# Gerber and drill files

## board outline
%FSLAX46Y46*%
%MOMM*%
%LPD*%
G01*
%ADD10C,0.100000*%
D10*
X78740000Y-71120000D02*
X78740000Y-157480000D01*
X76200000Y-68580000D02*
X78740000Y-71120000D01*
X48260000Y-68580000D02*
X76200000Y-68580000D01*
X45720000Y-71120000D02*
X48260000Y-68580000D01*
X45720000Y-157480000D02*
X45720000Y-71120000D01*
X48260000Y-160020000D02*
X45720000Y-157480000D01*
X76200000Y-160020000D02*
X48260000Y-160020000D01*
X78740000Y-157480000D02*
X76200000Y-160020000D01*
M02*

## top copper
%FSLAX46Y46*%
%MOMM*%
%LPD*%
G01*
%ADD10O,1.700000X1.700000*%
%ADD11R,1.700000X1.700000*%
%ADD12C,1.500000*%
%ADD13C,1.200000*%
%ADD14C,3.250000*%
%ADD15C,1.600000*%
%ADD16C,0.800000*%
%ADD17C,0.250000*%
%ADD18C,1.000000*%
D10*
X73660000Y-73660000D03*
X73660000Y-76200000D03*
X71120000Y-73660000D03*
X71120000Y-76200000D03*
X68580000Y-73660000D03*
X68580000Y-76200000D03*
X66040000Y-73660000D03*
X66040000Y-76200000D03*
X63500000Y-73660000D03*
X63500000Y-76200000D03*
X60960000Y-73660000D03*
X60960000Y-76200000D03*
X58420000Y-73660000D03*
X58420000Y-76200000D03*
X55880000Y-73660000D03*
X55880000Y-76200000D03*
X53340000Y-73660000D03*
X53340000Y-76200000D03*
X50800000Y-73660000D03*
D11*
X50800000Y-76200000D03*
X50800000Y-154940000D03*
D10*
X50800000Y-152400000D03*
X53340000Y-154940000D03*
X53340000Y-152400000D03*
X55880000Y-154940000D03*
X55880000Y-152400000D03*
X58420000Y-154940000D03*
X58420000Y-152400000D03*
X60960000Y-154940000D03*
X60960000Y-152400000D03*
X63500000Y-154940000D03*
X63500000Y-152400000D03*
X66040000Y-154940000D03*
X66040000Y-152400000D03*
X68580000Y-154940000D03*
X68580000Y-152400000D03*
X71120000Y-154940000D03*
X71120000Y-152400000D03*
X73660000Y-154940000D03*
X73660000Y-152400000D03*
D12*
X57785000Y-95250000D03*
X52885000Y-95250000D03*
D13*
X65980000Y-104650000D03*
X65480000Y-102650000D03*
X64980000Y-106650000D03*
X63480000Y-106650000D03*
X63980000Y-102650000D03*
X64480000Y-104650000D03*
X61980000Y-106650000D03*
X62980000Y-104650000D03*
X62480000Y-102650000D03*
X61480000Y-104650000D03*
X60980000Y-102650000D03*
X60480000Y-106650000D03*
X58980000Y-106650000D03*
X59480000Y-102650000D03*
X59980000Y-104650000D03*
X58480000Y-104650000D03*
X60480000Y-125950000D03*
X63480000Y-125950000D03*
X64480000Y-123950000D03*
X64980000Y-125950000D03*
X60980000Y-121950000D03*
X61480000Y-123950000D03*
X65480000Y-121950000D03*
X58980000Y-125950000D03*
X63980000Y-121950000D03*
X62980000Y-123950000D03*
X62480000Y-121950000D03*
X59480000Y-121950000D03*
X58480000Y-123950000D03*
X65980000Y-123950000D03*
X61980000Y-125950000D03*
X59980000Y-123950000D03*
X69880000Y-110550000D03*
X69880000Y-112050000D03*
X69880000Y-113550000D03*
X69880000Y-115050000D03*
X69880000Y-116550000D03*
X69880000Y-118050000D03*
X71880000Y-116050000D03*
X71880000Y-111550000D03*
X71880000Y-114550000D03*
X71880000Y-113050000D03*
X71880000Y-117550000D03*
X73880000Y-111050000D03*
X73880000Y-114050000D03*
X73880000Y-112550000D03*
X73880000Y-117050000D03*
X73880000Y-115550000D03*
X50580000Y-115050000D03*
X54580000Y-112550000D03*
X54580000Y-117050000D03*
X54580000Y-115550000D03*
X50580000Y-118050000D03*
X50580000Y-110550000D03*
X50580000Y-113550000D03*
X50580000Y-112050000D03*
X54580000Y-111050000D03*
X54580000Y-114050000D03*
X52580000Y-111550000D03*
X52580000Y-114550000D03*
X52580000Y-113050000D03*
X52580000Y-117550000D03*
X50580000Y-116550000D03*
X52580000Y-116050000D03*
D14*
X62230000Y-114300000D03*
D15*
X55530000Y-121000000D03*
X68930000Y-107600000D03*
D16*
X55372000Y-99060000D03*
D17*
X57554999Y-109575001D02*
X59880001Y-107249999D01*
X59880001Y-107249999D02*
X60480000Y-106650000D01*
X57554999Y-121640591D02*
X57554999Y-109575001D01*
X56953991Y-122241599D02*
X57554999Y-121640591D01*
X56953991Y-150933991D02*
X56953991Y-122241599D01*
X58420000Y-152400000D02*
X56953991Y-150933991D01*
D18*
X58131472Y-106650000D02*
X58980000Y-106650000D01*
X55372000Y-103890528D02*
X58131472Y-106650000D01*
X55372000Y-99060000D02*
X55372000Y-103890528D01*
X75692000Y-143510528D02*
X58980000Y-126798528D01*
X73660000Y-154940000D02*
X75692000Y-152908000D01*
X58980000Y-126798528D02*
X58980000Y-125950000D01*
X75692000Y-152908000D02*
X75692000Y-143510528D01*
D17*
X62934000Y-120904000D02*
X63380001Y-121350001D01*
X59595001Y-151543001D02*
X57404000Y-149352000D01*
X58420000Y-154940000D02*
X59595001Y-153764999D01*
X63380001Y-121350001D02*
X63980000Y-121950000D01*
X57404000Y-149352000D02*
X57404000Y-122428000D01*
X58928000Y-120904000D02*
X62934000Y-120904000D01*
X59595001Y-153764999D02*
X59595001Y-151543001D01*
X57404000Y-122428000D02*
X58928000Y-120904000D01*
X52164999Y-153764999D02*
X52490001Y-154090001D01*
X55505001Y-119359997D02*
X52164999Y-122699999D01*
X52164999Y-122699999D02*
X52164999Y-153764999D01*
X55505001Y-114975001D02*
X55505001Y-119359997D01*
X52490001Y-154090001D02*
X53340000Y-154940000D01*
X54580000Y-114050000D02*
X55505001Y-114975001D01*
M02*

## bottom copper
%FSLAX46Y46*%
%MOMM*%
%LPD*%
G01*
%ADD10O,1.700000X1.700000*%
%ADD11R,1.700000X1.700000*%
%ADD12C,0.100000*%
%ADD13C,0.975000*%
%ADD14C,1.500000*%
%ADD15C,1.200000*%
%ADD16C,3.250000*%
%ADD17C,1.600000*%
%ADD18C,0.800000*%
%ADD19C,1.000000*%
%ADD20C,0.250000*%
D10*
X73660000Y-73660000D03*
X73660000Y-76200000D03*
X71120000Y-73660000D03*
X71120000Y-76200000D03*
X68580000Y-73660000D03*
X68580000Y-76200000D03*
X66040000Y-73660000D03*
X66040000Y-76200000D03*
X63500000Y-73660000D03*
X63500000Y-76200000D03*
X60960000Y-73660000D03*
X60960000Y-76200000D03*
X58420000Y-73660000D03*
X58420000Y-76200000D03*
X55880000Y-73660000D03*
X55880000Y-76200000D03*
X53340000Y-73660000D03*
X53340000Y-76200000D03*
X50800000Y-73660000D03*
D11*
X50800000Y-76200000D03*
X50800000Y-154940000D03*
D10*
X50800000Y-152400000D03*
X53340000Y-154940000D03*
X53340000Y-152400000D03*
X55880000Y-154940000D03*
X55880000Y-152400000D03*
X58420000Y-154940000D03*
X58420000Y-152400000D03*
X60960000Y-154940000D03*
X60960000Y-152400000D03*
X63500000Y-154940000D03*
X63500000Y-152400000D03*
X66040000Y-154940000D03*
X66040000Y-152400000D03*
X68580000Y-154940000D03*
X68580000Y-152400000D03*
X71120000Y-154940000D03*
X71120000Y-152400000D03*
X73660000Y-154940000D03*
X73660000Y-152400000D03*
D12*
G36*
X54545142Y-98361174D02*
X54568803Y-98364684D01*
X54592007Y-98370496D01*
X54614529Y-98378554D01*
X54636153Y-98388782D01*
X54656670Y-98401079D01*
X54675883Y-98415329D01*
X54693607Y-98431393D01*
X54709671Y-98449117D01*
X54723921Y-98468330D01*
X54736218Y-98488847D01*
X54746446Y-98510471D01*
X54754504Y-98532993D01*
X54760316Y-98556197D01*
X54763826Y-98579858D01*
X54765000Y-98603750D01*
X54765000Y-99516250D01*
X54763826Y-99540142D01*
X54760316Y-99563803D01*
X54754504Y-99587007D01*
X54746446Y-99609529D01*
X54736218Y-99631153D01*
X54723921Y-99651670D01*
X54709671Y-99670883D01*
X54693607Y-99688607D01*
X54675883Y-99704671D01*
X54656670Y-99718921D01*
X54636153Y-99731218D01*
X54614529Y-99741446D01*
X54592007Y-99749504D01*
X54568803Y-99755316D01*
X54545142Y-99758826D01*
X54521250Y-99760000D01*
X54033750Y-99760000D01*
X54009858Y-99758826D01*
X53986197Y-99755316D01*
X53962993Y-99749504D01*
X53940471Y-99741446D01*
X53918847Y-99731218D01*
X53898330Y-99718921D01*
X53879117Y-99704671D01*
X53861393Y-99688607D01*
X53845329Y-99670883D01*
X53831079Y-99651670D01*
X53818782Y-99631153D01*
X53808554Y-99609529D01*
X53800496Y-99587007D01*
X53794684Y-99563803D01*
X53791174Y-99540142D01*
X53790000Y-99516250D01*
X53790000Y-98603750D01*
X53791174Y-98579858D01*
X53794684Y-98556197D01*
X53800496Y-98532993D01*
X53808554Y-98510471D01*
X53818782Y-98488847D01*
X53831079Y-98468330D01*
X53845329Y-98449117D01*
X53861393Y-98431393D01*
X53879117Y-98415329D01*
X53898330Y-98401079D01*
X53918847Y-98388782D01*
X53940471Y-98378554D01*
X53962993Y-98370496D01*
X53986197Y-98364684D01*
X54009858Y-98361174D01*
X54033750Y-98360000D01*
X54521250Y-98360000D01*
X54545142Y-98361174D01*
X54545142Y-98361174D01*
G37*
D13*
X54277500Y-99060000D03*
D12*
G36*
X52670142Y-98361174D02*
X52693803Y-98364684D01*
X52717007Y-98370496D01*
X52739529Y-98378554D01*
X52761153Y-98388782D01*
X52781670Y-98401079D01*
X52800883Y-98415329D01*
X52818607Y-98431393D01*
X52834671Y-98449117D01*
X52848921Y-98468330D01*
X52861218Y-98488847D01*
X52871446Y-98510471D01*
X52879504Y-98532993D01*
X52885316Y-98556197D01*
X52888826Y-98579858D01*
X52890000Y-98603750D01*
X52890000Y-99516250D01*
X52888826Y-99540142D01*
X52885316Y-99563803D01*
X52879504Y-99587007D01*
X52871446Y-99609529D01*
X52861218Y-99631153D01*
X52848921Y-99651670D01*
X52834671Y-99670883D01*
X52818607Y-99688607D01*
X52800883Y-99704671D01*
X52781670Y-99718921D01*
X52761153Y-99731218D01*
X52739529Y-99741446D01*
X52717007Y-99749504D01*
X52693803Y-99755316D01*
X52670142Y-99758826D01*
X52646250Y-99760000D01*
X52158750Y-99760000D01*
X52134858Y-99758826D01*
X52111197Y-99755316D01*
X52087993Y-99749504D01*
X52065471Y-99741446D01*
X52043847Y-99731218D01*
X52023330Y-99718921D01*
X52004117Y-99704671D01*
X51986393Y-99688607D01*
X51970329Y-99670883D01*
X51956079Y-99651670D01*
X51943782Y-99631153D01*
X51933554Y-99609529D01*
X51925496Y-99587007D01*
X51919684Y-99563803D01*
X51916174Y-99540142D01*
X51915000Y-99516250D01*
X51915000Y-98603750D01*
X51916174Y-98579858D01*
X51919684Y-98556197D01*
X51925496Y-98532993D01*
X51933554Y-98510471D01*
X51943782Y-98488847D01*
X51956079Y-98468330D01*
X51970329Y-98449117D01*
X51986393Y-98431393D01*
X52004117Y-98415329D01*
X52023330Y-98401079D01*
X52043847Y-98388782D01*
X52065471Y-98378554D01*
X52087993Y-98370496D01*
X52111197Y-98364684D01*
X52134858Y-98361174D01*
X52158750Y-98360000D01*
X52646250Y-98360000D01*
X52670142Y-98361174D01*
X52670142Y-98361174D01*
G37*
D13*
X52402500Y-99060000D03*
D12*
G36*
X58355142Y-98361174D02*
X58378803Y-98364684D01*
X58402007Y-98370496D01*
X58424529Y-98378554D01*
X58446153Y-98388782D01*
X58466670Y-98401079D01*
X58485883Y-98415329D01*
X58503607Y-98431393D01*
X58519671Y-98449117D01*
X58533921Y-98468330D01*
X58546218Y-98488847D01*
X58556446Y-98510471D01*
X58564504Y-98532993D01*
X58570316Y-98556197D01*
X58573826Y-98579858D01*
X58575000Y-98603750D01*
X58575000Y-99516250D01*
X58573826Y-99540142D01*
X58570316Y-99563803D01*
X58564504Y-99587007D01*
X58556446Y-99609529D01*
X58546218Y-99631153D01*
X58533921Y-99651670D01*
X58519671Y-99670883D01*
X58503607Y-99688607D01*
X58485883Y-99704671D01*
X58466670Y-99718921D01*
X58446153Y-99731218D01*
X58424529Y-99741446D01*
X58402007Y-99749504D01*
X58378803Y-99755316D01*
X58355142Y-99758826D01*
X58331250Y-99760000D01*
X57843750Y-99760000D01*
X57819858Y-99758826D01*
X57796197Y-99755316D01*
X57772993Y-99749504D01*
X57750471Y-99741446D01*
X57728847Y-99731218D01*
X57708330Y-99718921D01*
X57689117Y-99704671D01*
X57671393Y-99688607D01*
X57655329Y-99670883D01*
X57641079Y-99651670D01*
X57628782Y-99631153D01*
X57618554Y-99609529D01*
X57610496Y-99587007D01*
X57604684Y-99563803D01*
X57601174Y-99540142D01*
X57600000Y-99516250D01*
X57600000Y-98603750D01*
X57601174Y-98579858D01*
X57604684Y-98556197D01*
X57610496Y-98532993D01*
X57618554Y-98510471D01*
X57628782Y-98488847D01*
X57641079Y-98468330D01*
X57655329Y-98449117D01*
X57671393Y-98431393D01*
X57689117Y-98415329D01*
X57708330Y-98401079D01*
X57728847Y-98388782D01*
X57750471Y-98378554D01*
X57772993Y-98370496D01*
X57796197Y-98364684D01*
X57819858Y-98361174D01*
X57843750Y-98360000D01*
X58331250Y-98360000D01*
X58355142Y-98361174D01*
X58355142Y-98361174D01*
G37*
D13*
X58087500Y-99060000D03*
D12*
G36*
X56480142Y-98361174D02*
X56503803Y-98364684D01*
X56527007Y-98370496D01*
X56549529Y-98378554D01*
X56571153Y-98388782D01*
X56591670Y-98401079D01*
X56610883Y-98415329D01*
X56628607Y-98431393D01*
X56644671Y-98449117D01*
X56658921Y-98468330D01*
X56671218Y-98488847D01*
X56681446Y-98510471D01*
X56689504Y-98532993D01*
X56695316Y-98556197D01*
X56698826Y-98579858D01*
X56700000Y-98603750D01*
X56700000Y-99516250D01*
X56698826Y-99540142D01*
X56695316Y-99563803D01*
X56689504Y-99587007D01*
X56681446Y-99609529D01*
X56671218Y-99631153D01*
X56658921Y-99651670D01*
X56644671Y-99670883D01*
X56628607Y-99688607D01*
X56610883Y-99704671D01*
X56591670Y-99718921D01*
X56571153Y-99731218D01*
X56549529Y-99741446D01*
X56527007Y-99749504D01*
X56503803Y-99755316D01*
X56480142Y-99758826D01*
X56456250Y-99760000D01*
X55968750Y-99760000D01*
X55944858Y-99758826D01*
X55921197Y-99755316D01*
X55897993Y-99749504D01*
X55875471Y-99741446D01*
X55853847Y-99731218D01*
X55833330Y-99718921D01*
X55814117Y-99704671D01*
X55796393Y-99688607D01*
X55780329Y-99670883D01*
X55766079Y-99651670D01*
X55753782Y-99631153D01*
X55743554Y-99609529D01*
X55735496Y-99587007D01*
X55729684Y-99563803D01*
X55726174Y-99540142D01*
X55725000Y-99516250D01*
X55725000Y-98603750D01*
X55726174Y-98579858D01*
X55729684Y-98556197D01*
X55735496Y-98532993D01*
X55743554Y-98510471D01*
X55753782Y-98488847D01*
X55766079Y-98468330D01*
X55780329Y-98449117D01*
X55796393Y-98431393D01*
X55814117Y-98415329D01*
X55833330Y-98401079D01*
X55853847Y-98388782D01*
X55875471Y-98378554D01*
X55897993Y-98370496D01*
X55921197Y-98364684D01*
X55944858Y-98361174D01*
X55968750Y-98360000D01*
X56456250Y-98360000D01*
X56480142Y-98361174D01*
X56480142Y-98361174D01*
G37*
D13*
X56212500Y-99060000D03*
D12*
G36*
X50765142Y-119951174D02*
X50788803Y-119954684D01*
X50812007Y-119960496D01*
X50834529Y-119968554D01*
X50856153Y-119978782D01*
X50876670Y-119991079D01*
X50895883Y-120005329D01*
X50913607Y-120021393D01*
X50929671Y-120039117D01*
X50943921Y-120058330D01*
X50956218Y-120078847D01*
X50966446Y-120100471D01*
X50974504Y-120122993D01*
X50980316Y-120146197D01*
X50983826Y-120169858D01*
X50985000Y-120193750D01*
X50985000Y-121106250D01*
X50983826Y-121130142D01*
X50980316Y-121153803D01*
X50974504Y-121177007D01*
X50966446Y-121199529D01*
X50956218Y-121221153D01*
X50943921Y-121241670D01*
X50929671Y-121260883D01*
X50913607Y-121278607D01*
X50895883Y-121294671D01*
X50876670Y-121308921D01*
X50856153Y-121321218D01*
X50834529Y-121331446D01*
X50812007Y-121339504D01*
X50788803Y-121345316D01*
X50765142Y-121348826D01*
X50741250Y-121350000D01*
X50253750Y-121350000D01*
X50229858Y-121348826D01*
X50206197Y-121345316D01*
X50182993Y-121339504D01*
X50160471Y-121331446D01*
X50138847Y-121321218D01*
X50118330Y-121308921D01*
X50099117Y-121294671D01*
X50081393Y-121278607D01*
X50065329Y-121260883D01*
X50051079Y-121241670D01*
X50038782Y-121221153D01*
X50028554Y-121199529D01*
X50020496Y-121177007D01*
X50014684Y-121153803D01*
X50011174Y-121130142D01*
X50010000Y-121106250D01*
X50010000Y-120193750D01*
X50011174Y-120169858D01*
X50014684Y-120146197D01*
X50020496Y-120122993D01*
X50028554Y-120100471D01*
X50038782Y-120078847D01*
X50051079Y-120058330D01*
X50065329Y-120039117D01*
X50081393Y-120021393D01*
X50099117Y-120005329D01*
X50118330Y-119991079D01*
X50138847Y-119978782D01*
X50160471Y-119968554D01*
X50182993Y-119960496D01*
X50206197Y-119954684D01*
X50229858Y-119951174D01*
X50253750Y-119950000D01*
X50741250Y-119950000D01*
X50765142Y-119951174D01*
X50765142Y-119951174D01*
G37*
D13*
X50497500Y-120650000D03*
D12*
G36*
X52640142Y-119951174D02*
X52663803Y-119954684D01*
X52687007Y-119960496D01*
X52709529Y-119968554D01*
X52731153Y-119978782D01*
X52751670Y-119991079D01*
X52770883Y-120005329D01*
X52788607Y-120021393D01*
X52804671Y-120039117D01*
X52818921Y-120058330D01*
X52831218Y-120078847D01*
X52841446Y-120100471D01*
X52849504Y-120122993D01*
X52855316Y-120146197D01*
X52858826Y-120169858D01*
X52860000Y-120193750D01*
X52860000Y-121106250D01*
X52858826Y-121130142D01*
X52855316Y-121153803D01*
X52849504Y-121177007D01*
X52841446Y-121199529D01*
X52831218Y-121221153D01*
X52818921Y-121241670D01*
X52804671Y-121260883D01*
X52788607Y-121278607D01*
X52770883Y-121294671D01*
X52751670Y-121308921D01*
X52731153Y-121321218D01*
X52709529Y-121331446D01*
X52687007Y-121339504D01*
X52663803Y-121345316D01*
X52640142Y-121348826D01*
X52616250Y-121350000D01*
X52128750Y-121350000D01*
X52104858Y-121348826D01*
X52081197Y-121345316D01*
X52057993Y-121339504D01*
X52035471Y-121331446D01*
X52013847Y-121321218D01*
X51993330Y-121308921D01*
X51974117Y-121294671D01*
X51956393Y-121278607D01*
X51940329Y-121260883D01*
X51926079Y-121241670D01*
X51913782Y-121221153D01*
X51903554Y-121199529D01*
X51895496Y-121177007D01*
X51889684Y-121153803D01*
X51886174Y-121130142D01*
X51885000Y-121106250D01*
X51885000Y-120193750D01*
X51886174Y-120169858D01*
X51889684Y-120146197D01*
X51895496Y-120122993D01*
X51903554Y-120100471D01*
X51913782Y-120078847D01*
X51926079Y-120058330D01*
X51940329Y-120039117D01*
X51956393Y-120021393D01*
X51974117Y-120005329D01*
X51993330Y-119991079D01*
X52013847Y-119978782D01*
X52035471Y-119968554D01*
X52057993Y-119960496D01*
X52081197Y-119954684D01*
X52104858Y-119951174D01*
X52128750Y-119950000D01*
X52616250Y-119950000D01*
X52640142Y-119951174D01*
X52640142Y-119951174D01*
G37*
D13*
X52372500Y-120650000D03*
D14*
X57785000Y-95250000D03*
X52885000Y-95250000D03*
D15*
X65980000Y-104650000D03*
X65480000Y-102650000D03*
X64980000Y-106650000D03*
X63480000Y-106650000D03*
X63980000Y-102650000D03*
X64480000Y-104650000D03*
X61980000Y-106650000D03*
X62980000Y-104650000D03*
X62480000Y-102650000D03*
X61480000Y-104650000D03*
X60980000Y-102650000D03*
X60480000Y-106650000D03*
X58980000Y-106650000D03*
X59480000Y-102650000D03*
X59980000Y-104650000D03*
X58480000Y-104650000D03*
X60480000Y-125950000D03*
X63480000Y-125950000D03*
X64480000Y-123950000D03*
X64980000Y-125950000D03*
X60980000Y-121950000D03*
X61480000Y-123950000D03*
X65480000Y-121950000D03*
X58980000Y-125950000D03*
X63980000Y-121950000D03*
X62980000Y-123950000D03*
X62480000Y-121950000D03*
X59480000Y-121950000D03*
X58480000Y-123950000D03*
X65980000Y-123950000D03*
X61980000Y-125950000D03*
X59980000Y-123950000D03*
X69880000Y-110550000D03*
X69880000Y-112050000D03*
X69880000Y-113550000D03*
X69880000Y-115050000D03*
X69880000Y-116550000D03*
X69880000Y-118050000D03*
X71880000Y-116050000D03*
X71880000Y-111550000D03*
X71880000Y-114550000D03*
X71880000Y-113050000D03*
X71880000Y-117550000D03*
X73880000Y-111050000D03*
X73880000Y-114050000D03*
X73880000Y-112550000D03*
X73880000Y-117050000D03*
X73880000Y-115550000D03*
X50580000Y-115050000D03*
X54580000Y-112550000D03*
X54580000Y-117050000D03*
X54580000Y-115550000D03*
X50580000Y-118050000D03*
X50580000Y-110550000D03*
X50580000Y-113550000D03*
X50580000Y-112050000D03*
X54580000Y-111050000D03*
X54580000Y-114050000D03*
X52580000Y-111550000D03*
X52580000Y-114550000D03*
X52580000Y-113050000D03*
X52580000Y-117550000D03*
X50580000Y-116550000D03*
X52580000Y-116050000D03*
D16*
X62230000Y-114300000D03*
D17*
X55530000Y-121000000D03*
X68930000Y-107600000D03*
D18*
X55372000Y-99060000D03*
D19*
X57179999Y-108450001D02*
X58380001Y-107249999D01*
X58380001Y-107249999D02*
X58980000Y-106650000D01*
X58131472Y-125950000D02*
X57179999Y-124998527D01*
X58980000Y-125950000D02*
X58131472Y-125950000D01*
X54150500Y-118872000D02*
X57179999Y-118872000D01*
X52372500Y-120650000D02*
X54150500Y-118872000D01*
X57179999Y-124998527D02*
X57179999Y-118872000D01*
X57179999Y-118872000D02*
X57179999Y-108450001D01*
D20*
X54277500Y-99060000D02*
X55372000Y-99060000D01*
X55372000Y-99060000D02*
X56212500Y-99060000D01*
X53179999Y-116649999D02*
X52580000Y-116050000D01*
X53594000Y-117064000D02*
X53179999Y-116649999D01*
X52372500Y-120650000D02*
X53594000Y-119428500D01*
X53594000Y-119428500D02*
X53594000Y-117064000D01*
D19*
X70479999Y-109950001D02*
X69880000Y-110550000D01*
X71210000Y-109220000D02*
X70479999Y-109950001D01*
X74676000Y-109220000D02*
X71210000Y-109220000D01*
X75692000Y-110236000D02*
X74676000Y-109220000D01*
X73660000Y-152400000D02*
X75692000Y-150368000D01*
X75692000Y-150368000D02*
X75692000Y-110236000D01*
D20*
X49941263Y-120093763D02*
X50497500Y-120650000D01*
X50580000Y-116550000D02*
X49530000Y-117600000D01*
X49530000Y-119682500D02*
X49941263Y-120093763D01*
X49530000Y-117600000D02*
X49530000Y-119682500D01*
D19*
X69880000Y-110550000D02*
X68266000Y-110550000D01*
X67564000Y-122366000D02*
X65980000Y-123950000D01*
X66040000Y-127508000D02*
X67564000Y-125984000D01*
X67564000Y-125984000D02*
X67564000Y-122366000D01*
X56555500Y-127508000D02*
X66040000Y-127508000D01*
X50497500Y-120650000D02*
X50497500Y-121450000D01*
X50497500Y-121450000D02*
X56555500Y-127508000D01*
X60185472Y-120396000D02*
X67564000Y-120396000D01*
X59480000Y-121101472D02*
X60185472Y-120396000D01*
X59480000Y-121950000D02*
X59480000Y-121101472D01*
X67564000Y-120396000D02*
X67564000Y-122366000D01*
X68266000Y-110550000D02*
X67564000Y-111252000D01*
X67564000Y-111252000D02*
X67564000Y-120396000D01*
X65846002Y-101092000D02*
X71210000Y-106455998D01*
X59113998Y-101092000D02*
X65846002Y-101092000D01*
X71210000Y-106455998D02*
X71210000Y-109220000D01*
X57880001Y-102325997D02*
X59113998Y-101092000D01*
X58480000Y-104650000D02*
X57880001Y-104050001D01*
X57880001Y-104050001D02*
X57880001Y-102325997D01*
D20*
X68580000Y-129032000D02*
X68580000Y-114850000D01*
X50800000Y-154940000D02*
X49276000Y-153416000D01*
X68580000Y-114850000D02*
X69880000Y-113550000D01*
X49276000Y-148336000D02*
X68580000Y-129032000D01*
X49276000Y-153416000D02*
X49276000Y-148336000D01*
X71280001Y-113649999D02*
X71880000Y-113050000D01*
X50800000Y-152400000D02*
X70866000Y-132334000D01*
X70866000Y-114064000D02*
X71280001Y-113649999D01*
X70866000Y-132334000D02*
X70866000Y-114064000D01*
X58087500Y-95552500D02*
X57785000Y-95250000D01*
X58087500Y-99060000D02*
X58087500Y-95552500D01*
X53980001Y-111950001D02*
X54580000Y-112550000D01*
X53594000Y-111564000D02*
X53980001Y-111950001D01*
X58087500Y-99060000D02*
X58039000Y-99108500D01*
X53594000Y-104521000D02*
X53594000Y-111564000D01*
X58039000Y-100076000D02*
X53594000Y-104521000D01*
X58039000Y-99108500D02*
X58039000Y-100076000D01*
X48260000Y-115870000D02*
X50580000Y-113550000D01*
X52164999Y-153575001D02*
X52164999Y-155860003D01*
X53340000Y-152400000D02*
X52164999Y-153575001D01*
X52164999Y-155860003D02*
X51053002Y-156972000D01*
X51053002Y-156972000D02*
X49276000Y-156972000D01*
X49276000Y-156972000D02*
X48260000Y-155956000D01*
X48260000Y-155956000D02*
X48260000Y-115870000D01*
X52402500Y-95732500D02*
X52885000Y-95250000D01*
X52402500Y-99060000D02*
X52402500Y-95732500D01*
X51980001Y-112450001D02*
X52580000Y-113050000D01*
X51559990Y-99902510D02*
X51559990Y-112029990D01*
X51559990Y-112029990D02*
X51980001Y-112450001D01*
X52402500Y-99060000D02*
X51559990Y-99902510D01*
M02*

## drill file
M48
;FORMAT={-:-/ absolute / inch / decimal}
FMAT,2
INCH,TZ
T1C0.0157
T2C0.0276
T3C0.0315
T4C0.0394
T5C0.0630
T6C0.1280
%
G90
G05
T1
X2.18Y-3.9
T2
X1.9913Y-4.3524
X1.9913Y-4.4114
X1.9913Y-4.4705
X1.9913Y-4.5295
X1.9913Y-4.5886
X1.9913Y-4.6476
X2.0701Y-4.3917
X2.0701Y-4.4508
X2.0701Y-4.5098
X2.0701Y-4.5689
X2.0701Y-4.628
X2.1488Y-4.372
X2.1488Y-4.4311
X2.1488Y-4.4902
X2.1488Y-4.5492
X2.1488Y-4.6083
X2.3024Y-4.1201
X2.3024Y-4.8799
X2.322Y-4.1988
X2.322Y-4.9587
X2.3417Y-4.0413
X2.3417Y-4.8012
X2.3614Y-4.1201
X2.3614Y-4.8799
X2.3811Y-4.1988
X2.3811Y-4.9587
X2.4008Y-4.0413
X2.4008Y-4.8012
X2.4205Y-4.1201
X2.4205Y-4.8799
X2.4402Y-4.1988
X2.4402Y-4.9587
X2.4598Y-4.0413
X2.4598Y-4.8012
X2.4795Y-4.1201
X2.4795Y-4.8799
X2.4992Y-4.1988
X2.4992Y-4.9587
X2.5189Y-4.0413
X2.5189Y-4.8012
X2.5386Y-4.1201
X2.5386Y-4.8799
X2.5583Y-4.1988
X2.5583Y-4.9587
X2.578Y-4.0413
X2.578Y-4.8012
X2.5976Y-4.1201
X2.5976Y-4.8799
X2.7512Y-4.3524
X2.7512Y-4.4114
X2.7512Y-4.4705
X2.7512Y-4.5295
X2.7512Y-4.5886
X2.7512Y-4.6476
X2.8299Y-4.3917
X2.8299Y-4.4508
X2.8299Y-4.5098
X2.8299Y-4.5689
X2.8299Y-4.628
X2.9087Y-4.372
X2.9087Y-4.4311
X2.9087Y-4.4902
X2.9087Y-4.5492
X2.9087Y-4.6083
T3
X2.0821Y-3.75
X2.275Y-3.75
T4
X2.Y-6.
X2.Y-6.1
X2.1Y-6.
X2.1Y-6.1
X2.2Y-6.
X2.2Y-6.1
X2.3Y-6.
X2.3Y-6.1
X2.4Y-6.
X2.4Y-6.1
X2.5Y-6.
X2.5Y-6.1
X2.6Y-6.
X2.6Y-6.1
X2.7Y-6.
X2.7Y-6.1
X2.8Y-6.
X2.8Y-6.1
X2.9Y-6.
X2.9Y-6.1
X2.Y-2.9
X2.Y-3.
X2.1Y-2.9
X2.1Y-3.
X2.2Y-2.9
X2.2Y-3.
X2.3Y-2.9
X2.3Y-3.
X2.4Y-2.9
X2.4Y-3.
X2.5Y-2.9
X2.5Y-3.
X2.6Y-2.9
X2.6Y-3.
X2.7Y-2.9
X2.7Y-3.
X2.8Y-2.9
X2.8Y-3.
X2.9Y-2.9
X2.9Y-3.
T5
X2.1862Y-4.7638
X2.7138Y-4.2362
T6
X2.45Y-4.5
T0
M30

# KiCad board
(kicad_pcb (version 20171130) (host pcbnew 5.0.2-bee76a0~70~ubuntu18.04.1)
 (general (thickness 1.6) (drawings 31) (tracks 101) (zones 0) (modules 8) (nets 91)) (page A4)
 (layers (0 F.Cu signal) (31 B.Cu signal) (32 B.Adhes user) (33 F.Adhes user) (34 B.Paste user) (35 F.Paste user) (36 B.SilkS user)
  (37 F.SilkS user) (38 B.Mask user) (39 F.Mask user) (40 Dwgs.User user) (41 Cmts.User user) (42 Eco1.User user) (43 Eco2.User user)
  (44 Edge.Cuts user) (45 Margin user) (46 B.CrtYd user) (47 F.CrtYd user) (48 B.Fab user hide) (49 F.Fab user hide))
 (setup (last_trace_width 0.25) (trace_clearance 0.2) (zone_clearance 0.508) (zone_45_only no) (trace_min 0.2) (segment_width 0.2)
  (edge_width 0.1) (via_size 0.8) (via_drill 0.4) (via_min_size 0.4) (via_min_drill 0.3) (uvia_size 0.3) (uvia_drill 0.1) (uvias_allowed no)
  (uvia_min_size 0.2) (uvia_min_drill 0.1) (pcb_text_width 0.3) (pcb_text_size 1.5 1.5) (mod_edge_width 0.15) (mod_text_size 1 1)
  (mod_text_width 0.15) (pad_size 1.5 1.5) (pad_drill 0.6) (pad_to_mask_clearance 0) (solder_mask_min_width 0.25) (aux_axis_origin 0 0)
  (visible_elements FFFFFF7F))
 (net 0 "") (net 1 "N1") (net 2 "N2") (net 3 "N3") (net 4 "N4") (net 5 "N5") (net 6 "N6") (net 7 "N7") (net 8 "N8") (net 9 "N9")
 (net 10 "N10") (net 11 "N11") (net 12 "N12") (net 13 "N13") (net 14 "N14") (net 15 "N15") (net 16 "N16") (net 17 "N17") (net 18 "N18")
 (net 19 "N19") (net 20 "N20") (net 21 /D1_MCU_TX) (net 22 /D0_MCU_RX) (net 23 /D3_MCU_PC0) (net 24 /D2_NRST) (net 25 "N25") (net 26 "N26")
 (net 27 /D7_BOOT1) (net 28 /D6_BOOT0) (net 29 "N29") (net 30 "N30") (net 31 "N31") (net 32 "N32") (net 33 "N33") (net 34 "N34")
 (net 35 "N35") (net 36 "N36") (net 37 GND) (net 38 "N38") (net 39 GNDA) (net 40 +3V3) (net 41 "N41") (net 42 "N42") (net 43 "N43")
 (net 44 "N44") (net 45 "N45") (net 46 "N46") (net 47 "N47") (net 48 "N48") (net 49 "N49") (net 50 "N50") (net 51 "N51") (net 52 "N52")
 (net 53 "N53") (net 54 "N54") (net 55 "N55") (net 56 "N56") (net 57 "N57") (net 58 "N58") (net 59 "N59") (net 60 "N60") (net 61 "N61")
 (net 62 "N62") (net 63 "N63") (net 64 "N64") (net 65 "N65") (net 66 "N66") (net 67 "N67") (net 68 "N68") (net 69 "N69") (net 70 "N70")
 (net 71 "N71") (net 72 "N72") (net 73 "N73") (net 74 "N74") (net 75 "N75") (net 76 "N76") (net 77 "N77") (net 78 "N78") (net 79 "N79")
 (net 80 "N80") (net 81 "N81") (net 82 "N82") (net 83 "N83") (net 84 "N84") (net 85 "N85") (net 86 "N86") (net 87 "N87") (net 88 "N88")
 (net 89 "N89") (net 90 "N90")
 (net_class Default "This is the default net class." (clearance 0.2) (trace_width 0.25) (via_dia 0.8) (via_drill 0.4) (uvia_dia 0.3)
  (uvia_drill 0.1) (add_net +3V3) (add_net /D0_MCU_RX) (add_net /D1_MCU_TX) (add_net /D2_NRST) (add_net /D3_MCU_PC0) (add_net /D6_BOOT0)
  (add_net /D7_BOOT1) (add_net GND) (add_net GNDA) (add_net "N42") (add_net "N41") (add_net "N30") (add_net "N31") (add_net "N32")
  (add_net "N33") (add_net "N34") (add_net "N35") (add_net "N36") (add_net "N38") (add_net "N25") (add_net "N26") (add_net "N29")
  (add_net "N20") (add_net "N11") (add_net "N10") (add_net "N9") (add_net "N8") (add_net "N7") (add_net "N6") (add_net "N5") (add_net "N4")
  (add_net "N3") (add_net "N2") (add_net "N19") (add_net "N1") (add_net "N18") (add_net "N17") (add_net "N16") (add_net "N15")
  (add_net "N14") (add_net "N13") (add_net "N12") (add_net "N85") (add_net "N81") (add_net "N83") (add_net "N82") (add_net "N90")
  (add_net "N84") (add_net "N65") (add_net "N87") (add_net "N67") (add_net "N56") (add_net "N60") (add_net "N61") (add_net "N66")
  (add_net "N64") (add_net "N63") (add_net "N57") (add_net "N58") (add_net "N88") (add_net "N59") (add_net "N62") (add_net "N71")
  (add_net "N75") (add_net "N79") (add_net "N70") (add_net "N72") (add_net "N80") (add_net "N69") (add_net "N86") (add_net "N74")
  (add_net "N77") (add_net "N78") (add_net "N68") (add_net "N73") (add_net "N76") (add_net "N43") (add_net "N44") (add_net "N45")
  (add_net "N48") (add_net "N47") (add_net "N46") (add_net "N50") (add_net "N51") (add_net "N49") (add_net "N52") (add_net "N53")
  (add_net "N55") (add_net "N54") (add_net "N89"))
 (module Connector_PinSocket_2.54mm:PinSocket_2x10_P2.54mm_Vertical (layer B.Cu) (at 50.8 76.2 270)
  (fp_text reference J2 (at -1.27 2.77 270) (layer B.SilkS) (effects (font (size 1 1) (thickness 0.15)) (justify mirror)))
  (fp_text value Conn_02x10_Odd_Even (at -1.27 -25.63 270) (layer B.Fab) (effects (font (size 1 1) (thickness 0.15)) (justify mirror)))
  (pad 20 thru_hole oval (at -2.54 -22.86 270) (size 1.7 1.7) (drill 1) (layers *.Cu *.Mask) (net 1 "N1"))
  (pad 19 thru_hole oval (at 0 -22.86 270) (size 1.7 1.7) (drill 1) (layers *.Cu *.Mask) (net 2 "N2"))
  (pad 18 thru_hole oval (at -2.54 -20.32 270) (size 1.7 1.7) (drill 1) (layers *.Cu *.Mask) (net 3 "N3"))
  (pad 17 thru_hole oval (at 0 -20.32 270) (size 1.7 1.7) (drill 1) (layers *.Cu *.Mask) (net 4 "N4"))
  (pad 16 thru_hole oval (at -2.54 -17.78 270) (size 1.7 1.7) (drill 1) (layers *.Cu *.Mask) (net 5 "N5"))
  (pad 15 thru_hole oval (at 0 -17.78 270) (size 1.7 1.7) (drill 1) (layers *.Cu *.Mask) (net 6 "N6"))
  (pad 14 thru_hole oval (at -2.54 -15.24 270) (size 1.7 1.7) (drill 1) (layers *.Cu *.Mask) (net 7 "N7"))
  (pad 13 thru_hole oval (at 0 -15.24 270) (size 1.7 1.7) (drill 1) (layers *.Cu *.Mask) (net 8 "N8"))
  (pad 12 thru_hole oval (at -2.54 -12.7 270) (size 1.7 1.7) (drill 1) (layers *.Cu *.Mask) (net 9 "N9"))
  (pad 11 thru_hole oval (at 0 -12.7 270) (size 1.7 1.7) (drill 1) (layers *.Cu *.Mask) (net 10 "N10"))
  (pad 10 thru_hole oval (at -2.54 -10.16 270) (size 1.7 1.7) (drill 1) (layers *.Cu *.Mask) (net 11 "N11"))
  (pad 9 thru_hole oval (at 0 -10.16 270) (size 1.7 1.7) (drill 1) (layers *.Cu *.Mask) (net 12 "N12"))
  (pad 8 thru_hole oval (at -2.54 -7.62 270) (size 1.7 1.7) (drill 1) (layers *.Cu *.Mask) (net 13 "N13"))
  (pad 7 thru_hole oval (at 0 -7.62 270) (size 1.7 1.7) (drill 1) (layers *.Cu *.Mask) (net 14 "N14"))
  (pad 6 thru_hole oval (at -2.54 -5.08 270) (size 1.7 1.7) (drill 1) (layers *.Cu *.Mask) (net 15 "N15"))
  (pad 5 thru_hole oval (at 0 -5.08 270) (size 1.7 1.7) (drill 1) (layers *.Cu *.Mask) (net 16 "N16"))
  (pad 4 thru_hole oval (at -2.54 -2.54 270) (size 1.7 1.7) (drill 1) (layers *.Cu *.Mask) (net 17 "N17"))
  (pad 3 thru_hole oval (at 0 -2.54 270) (size 1.7 1.7) (drill 1) (layers *.Cu *.Mask) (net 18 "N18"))
  (pad 2 thru_hole oval (at -2.54 0 270) (size 1.7 1.7) (drill 1) (layers *.Cu *.Mask) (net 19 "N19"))
  (pad 1 thru_hole rect (at 0 0 270) (size 1.7 1.7) (drill 1) (layers *.Cu *.Mask) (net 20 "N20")))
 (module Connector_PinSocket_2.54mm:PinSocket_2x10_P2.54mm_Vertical (layer B.Cu) (at 50.8 154.94 270)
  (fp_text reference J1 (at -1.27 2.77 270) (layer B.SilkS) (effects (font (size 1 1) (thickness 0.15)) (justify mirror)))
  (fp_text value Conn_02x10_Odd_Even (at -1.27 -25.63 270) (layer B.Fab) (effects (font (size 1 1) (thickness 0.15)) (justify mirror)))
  (pad 1 thru_hole rect (at 0 0 270) (size 1.7 1.7) (drill 1) (layers *.Cu *.Mask) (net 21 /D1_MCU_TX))
  (pad 2 thru_hole oval (at -2.54 0 270) (size 1.7 1.7) (drill 1) (layers *.Cu *.Mask) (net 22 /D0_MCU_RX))
  (pad 3 thru_hole oval (at 0 -2.54 270) (size 1.7 1.7) (drill 1) (layers *.Cu *.Mask) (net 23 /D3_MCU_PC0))
  (pad 4 thru_hole oval (at -2.54 -2.54 270) (size 1.7 1.7) (drill 1) (layers *.Cu *.Mask) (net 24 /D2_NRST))
  (pad 5 thru_hole oval (at 0 -5.08 270) (size 1.7 1.7) (drill 1) (layers *.Cu *.Mask) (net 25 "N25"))
  (pad 6 thru_hole oval (at -2.54 -5.08 270) (size 1.7 1.7) (drill 1) (layers *.Cu *.Mask) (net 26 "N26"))
  (pad 7 thru_hole oval (at 0 -7.62 270) (size 1.7 1.7) (drill 1) (layers *.Cu *.Mask) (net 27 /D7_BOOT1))
  (pad 8 thru_hole oval (at -2.54 -7.62 270) (size 1.7 1.7) (drill 1) (layers *.Cu *.Mask) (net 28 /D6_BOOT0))
  (pad 9 thru_hole oval (at 0 -10.16 270) (size 1.7 1.7) (drill 1) (layers *.Cu *.Mask) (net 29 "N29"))
  (pad 10 thru_hole oval (at -2.54 -10.16 270) (size 1.7 1.7) (drill 1) (layers *.Cu *.Mask) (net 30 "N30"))
  (pad 11 thru_hole oval (at 0 -12.7 270) (size 1.7 1.7) (drill 1) (layers *.Cu *.Mask) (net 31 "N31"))
  (pad 12 thru_hole oval (at -2.54 -12.7 270) (size 1.7 1.7) (drill 1) (layers *.Cu *.Mask) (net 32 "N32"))
  (pad 13 thru_hole oval (at 0 -15.24 270) (size 1.7 1.7) (drill 1) (layers *.Cu *.Mask) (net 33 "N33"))
  (pad 14 thru_hole oval (at -2.54 -15.24 270) (size 1.7 1.7) (drill 1) (layers *.Cu *.Mask) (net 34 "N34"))
  (pad 15 thru_hole oval (at 0 -17.78 270) (size 1.7 1.7) (drill 1) (layers *.Cu *.Mask) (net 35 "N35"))
  (pad 16 thru_hole oval (at -2.54 -17.78 270) (size 1.7 1.7) (drill 1) (layers *.Cu *.Mask) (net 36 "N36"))
  (pad 17 thru_hole oval (at 0 -20.32 270) (size 1.7 1.7) (drill 1) (layers *.Cu *.Mask) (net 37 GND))
  (pad 18 thru_hole oval (at -2.54 -20.32 270) (size 1.7 1.7) (drill 1) (layers *.Cu *.Mask) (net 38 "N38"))
  (pad 19 thru_hole oval (at 0 -22.86 270) (size 1.7 1.7) (drill 1) (layers *.Cu *.Mask) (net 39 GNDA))
  (pad 20 thru_hole oval (at -2.54 -22.86 270) (size 1.7 1.7) (drill 1) (layers *.Cu *.Mask) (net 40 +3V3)))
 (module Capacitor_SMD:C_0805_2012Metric (layer B.Cu) (at 53.34 99.06 180)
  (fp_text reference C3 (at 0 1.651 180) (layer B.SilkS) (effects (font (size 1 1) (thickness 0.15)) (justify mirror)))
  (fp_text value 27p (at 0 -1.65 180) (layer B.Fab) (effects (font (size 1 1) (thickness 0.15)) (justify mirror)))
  (pad 1 smd roundrect (at -0.9375 0 180) (size 0.975 1.4) (layers B.Cu B.Paste B.Mask) (roundrect_rratio 0.25) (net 39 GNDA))
  (pad 2 smd roundrect (at 0.9375 0 180) (size 0.975 1.4) (layers B.Cu B.Paste B.Mask) (roundrect_rratio 0.25) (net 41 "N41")))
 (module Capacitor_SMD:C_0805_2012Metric (layer B.Cu) (at 57.15 99.06)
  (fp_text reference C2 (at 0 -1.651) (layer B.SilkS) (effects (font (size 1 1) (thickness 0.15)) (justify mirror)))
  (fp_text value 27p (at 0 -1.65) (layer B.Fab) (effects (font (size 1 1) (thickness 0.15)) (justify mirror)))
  (pad 2 smd roundrect (at 0.9375 0) (size 0.975 1.4) (layers B.Cu B.Paste B.Mask) (roundrect_rratio 0.25) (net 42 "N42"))
  (pad 1 smd roundrect (at -0.9375 0) (size 0.975 1.4) (layers B.Cu B.Paste B.Mask) (roundrect_rratio 0.25) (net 39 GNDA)))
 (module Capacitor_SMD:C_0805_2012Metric (layer B.Cu) (at 51.435 120.65)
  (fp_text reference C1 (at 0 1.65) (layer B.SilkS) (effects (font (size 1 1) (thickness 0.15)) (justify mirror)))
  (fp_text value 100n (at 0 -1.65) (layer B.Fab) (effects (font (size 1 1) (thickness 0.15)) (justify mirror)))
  (pad 1 smd roundrect (at -0.9375 0) (size 0.975 1.4) (layers B.Cu B.Paste B.Mask) (roundrect_rratio 0.25) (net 40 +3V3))
  (pad 2 smd roundrect (at 0.9375 0) (size 0.975 1.4) (layers B.Cu B.Paste B.Mask) (roundrect_rratio 0.25) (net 39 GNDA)))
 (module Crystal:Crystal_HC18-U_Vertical (layer F.Cu) (at 57.785 95.25 180)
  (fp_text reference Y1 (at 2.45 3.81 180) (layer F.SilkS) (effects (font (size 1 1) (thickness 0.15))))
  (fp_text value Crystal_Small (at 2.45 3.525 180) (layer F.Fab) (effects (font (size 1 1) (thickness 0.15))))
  (pad 1 thru_hole circle (at 0 0 180) (size 1.5 1.5) (drill 0.8) (layers *.Cu *.Mask) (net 42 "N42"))
  (pad 2 thru_hole circle (at 4.9 0 180) (size 1.5 1.5) (drill 0.8) (layers *.Cu *.Mask) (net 41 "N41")))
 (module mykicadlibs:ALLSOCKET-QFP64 (layer F.Cu) (at 62.23 114.3 180)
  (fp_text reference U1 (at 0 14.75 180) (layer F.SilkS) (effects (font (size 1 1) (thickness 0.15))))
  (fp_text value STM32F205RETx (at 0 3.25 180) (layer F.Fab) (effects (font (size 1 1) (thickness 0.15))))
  (pad 49 thru_hole circle (at -3.75 9.65 180) (size 1.2 1.2) (drill 0.7) (layers *.Cu *.Mask) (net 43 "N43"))
  (pad 50 thru_hole circle (at -3.25 11.65 180) (size 1.2 1.2) (drill 0.7) (layers *.Cu *.Mask) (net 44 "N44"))
  (pad 51 thru_hole circle (at -2.75 7.65 180) (size 1.2 1.2) (drill 0.7) (layers *.Cu *.Mask) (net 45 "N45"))
  (pad 54 thru_hole circle (at -1.25 7.65 180) (size 1.2 1.2) (drill 0.7) (layers *.Cu *.Mask) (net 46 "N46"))
  (pad 53 thru_hole circle (at -1.75 11.65 180) (size 1.2 1.2) (drill 0.7) (layers *.Cu *.Mask) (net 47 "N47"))
  (pad 52 thru_hole circle (at -2.25 9.65 180) (size 1.2 1.2) (drill 0.7) (layers *.Cu *.Mask) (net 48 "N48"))
  (pad 57 thru_hole circle (at 0.25 7.65 180) (size 1.2 1.2) (drill 0.7) (layers *.Cu *.Mask) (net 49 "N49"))
  (pad 55 thru_hole circle (at -0.75 9.65 180) (size 1.2 1.2) (drill 0.7) (layers *.Cu *.Mask) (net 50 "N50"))
  (pad 56 thru_hole circle (at -0.25 11.65 180) (size 1.2 1.2) (drill 0.7) (layers *.Cu *.Mask) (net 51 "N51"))
  (pad 58 thru_hole circle (at 0.75 9.65 180) (size 1.2 1.2) (drill 0.7) (layers *.Cu *.Mask) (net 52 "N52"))
  (pad 59 thru_hole circle (at 1.25 11.65 180) (size 1.2 1.2) (drill 0.7) (layers *.Cu *.Mask) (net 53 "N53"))
  (pad 60 thru_hole circle (at 1.75 7.65 180) (size 1.2 1.2) (drill 0.7) (layers *.Cu *.Mask) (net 28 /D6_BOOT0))
  (pad 63 thru_hole circle (at 3.25 7.65 180) (size 1.2 1.2) (drill 0.7) (layers *.Cu *.Mask) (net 39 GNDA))
  (pad 62 thru_hole circle (at 2.75 11.65 180) (size 1.2 1.2) (drill 0.7) (layers *.Cu *.Mask) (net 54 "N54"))
  (pad 61 thru_hole circle (at 2.25 9.65 180) (size 1.2 1.2) (drill 0.7) (layers *.Cu *.Mask) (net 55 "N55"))
  (pad 64 thru_hole circle (at 3.75 9.65 180) (size 1.2 1.2) (drill 0.7) (layers *.Cu *.Mask) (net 40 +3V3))
  (pad 21 thru_hole circle (at 1.75 -11.65 180) (size 1.2 1.2) (drill 0.7) (layers *.Cu *.Mask) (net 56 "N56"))
  (pad 27 thru_hole circle (at -1.25 -11.65 180) (size 1.2 1.2) (drill 0.7) (layers *.Cu *.Mask) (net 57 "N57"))
  (pad 29 thru_hole circle (at -2.25 -9.65 180) (size 1.2 1.2) (drill 0.7) (layers *.Cu *.Mask) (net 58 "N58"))
  (pad 30 thru_hole circle (at -2.75 -11.65 180) (size 1.2 1.2) (drill 0.7) (layers *.Cu *.Mask) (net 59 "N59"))
  (pad 22 thru_hole circle (at 1.25 -7.65 180) (size 1.2 1.2) (drill 0.7) (layers *.Cu *.Mask) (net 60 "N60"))
  (pad 23 thru_hole circle (at 0.75 -9.65 180) (size 1.2 1.2) (drill 0.7) (layers *.Cu *.Mask) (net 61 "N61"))
  (pad 31 thru_hole circle (at -3.25 -7.65 180) (size 1.2 1.2) (drill 0.7) (layers *.Cu *.Mask) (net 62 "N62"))
  (pad 18 thru_hole circle (at 3.25 -11.65 180) (size 1.2 1.2) (drill 0.7) (layers *.Cu *.Mask) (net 39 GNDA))
  (pad 28 thru_hole circle (at -1.75 -7.65 180) (size 1.2 1.2) (drill 0.7) (layers *.Cu *.Mask) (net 27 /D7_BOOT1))
  (pad 26 thru_hole circle (at -0.75 -9.65 180) (size 1.2 1.2) (drill 0.7) (layers *.Cu *.Mask) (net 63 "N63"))
  (pad 25 thru_hole circle (at -0.25 -7.65 180) (size 1.2 1.2) (drill 0.7) (layers *.Cu *.Mask) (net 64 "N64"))
  (pad 19 thru_hole circle (at 2.75 -7.65 180) (size 1.2 1.2) (drill 0.7) (layers *.Cu *.Mask) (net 40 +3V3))
  (pad 17 thru_hole circle (at 3.75 -9.65 180) (size 1.2 1.2) (drill 0.7) (layers *.Cu *.Mask) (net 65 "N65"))
  (pad 32 thru_hole circle (at -3.75 -9.65 180) (size 1.2 1.2) (drill 0.7) (layers *.Cu *.Mask) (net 40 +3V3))
  (pad 24 thru_hole circle (at 0.25 -11.65 180) (size 1.2 1.2) (drill 0.7) (layers *.Cu *.Mask) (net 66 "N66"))
  (pad 20 thru_hole circle (at 2.25 -9.65 180) (size 1.2 1.2) (drill 0.7) (layers *.Cu *.Mask) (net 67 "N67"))
  (pad 48 thru_hole circle (at -7.65 3.75 180) (size 1.2 1.2) (drill 0.7) (layers *.Cu *.Mask) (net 40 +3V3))
  (pad 45 thru_hole circle (at -7.65 2.25 180) (size 1.2 1.2) (drill 0.7) (layers *.Cu *.Mask) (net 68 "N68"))
  (pad 42 thru_hole circle (at -7.65 0.75 180) (size 1.2 1.2) (drill 0.7) (layers *.Cu *.Mask) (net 21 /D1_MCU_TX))
  (pad 39 thru_hole circle (at -7.65 -0.75 180) (size 1.2 1.2) (drill 0.7) (layers *.Cu *.Mask) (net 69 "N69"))
  (pad 36 thru_hole circle (at -7.65 -2.25 180) (size 1.2 1.2) (drill 0.7) (layers *.Cu *.Mask) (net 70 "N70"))
  (pad 33 thru_hole circle (at -7.65 -3.75 180) (size 1.2 1.2) (drill 0.7) (layers *.Cu *.Mask) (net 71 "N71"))
  (pad 37 thru_hole circle (at -9.65 -1.75 180) (size 1.2 1.2) (drill 0.7) (layers *.Cu *.Mask) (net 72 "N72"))
  (pad 46 thru_hole circle (at -9.65 2.75 180) (size 1.2 1.2) (drill 0.7) (layers *.Cu *.Mask) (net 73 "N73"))
  (pad 40 thru_hole circle (at -9.65 -0.25 180) (size 1.2 1.2) (drill 0.7) (layers *.Cu *.Mask) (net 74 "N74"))
  (pad 43 thru_hole circle (at -9.65 1.25 180) (size 1.2 1.2) (drill 0.7) (layers *.Cu *.Mask) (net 22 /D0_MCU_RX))
  (pad 34 thru_hole circle (at -9.65 -3.25 180) (size 1.2 1.2) (drill 0.7) (layers *.Cu *.Mask) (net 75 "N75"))
  (pad 47 thru_hole circle (at -11.65 3.25 180) (size 1.2 1.2) (drill 0.7) (layers *.Cu *.Mask) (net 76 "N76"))
  (pad 41 thru_hole circle (at -11.65 0.25 180) (size 1.2 1.2) (drill 0.7) (layers *.Cu *.Mask) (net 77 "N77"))
  (pad 44 thru_hole circle (at -11.65 1.75 180) (size 1.2 1.2) (drill 0.7) (layers *.Cu *.Mask) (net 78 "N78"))
  (pad 35 thru_hole circle (at -11.65 -2.75 180) (size 1.2 1.2) (drill 0.7) (layers *.Cu *.Mask) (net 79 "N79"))
  (pad 38 thru_hole circle (at -11.65 -1.25 180) (size 1.2 1.2) (drill 0.7) (layers *.Cu *.Mask) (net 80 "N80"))
  (pad 10 thru_hole circle (at 11.65 -0.75 180) (size 1.2 1.2) (drill 0.7) (layers *.Cu *.Mask) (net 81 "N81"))
  (pad 5 thru_hole circle (at 7.65 1.75 180) (size 1.2 1.2) (drill 0.7) (layers *.Cu *.Mask) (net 42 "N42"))
  (pad 14 thru_hole circle (at 7.65 -2.75 180) (size 1.2 1.2) (drill 0.7) (layers *.Cu *.Mask) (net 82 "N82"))
  (pad 11 thru_hole circle (at 7.65 -1.25 180) (size 1.2 1.2) (drill 0.7) (layers *.Cu *.Mask) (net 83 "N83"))
  (pad 16 thru_hole circle (at 11.65 -3.75 180) (size 1.2 1.2) (drill 0.7) (layers *.Cu *.Mask) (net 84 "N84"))
  (pad 1 thru_hole circle (at 11.65 3.75 180) (size 1.2 1.2) (drill 0.7) (layers *.Cu *.Mask) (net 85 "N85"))
  (pad 7 thru_hole circle (at 11.65 0.75 180) (size 1.2 1.2) (drill 0.7) (layers *.Cu *.Mask) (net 24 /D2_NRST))
  (pad 4 thru_hole circle (at 11.65 2.25 180) (size 1.2 1.2) (drill 0.7) (layers *.Cu *.Mask) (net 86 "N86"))
  (pad 2 thru_hole circle (at 7.65 3.25 180) (size 1.2 1.2) (drill 0.7) (layers *.Cu *.Mask) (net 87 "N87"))
  (pad 8 thru_hole circle (at 7.65 0.25 180) (size 1.2 1.2) (drill 0.7) (layers *.Cu *.Mask) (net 23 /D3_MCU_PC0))
  (pad 3 thru_hole circle (at 9.65 2.75 180) (size 1.2 1.2) (drill 0.7) (layers *.Cu *.Mask) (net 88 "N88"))
  (pad 9 thru_hole circle (at 9.65 -0.25 180) (size 1.2 1.2) (drill 0.7) (layers *.Cu *.Mask) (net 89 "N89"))
  (pad 6 thru_hole circle (at 9.65 1.25 180) (size 1.2 1.2) (drill 0.7) (layers *.Cu *.Mask) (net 41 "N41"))
  (pad 15 thru_hole circle (at 9.65 -3.25 180) (size 1.2 1.2) (drill 0.7) (layers *.Cu *.Mask) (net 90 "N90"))
  (pad 13 thru_hole circle (at 11.65 -2.25 180) (size 1.2 1.2) (drill 0.7) (layers *.Cu *.Mask) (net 40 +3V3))
  (pad 12 thru_hole circle (at 9.65 -1.75 180) (size 1.2 1.2) (drill 0.7) (layers *.Cu *.Mask) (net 39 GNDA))
  (pad ~ thru_hole circle (at 0 0 180) (size 3.25 3.25) (drill 3.25) (layers *.Cu *.Mask))
  (pad ~ thru_hole circle (at 6.7 -6.7 180) (size 1.6 1.6) (drill 1.6) (layers *.Cu *.Mask))
  (pad ~ thru_hole circle (at -6.7 6.7 180) (size 1.6 1.6) (drill 1.6) (layers *.Cu *.Mask)))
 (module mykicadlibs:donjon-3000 (layer F.Cu) (at 62.23 83.82)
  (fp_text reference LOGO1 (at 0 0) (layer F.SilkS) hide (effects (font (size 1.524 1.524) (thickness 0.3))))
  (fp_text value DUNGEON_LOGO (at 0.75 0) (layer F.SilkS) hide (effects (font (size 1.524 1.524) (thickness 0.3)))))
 (gr_line (start 78.74 71.12) (end 78.74 157.48) (layer Edge.Cuts) (width 0.1))
 (gr_line (start 76.2 68.58) (end 78.74 71.12) (layer Edge.Cuts) (width 0.1))
 (gr_line (start 48.26 68.58) (end 76.2 68.58) (layer Edge.Cuts) (width 0.1))
 (gr_line (start 45.72 71.12) (end 48.26 68.58) (layer Edge.Cuts) (width 0.1))
 (gr_line (start 45.72 157.48) (end 45.72 71.12) (layer Edge.Cuts) (width 0.1))
 (gr_line (start 48.26 160.02) (end 45.72 157.48) (layer Edge.Cuts) (width 0.1))
 (gr_line (start 76.2 160.02) (end 48.26 160.02) (layer Edge.Cuts) (width 0.1))
 (gr_line (start 78.74 157.48) (end 76.2 160.02) (layer Edge.Cuts) (width 0.1))
 (segment (start 57.554999 109.575001) (end 59.880001 107.249999) (width 0.25) (layer F.Cu) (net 28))
 (segment (start 59.880001 107.249999) (end 60.48 106.65) (width 0.25) (layer F.Cu) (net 28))
 (segment (start 57.554999 121.640591) (end 57.554999 109.575001) (width 0.25) (layer F.Cu) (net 28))
 (segment (start 56.953991 122.241599) (end 57.554999 121.640591) (width 0.25) (layer F.Cu) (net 28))
 (segment (start 56.953991 150.933991) (end 56.953991 122.241599) (width 0.25) (layer F.Cu) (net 28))
 (segment (start 58.42 152.4) (end 56.953991 150.933991) (width 0.25) (layer F.Cu) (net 28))
 (segment (start 57.179999 108.450001) (end 58.380001 107.249999) (width 1) (layer B.Cu) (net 39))
 (segment (start 58.380001 107.249999) (end 58.98 106.65) (width 1) (layer B.Cu) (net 39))
 (segment (start 58.131472 125.95) (end 57.179999 124.998527) (width 1) (layer B.Cu) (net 39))
 (segment (start 58.98 125.95) (end 58.131472 125.95) (width 1) (layer B.Cu) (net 39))
 (segment (start 54.1505 118.872) (end 57.179999 118.872) (width 1) (layer B.Cu) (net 39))
 (segment (start 52.3725 120.65) (end 54.1505 118.872) (width 1) (layer B.Cu) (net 39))
 (segment (start 57.179999 124.998527) (end 57.179999 118.872) (width 1) (layer B.Cu) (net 39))
 (segment (start 57.179999 118.872) (end 57.179999 108.450001) (width 1) (layer B.Cu) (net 39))
 (segment (start 54.2775 99.06) (end 55.372 99.06) (width 0.25) (layer B.Cu) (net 39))
 (via (at 55.372 99.06) (size 0.8) (drill 0.4) (layers F.Cu B.Cu) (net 39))
 (segment (start 55.372 99.06) (end 56.2125 99.06) (width 0.25) (layer B.Cu) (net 39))
 (segment (start 58.131472 106.65) (end 58.98 106.65) (width 1) (layer F.Cu) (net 39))
 (segment (start 55.372 103.890528) (end 58.131472 106.65) (width 1) (layer F.Cu) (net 39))
 (segment (start 55.372 99.06) (end 55.372 103.890528) (width 1) (layer F.Cu) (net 39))
 (segment (start 75.692 143.510528) (end 58.98 126.798528) (width 1) (layer F.Cu) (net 39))
 (segment (start 73.66 154.94) (end 75.692 152.908) (width 1) (layer F.Cu) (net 39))
 (segment (start 58.98 126.798528) (end 58.98 125.95) (width 1) (layer F.Cu) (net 39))
 (segment (start 75.692 152.908) (end 75.692 143.510528) (width 1) (layer F.Cu) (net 39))
 (segment (start 53.179999 116.649999) (end 52.58 116.05) (width 0.25) (layer B.Cu) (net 39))
 (segment (start 53.594 117.064) (end 53.179999 116.649999) (width 0.25) (layer B.Cu) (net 39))
 (segment (start 52.3725 120.65) (end 53.594 119.4285) (width 0.25) (layer B.Cu) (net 39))
 (segment (start 53.594 119.4285) (end 53.594 117.064) (width 0.25) (layer B.Cu) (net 39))
 (segment (start 70.479999 109.950001) (end 69.88 110.55) (width 1) (layer B.Cu) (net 40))
 (segment (start 71.21 109.22) (end 70.479999 109.950001) (width 1) (layer B.Cu) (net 40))
 (segment (start 74.676 109.22) (end 71.21 109.22) (width 1) (layer B.Cu) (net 40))
 (segment (start 75.692 110.236) (end 74.676 109.22) (width 1) (layer B.Cu) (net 40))
 (segment (start 73.66 152.4) (end 75.692 150.368) (width 1) (layer B.Cu) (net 40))
 (segment (start 75.692 150.368) (end 75.692 110.236) (width 1) (layer B.Cu) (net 40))
 (segment (start 49.941263 120.093763) (end 50.4975 120.65) (width 0.25) (layer B.Cu) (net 40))
 (segment (start 50.58 116.55) (end 49.53 117.6) (width 0.25) (layer B.Cu) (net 40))
 (segment (start 49.53 119.6825) (end 49.941263 120.093763) (width 0.25) (layer B.Cu) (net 40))
 (segment (start 49.53 117.6) (end 49.53 119.6825) (width 0.25) (layer B.Cu) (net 40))
 (segment (start 69.88 110.55) (end 68.266 110.55) (width 1) (layer B.Cu) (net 40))
 (segment (start 67.564 122.366) (end 65.98 123.95) (width 1) (layer B.Cu) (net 40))
 (segment (start 66.04 127.508) (end 67.564 125.984) (width 1) (layer B.Cu) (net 40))
 (segment (start 67.564 125.984) (end 67.564 122.366) (width 1) (layer B.Cu) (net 40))
 (segment (start 56.5555 127.508) (end 66.04 127.508) (width 1) (layer B.Cu) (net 40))
 (segment (start 50.4975 120.65) (end 50.4975 121.45) (width 1) (layer B.Cu) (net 40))
 (segment (start 50.4975 121.45) (end 56.5555 127.508) (width 1) (layer B.Cu) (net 40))
 (segment (start 60.185472 120.396) (end 67.564 120.396) (width 1) (layer B.Cu) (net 40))
 (segment (start 59.48 121.101472) (end 60.185472 120.396) (width 1) (layer B.Cu) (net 40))
 (segment (start 59.48 121.95) (end 59.48 121.101472) (width 1) (layer B.Cu) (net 40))
 (segment (start 67.564 120.396) (end 67.564 122.366) (width 1) (layer B.Cu) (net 40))
 (segment (start 68.266 110.55) (end 67.564 111.252) (width 1) (layer B.Cu) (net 40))
 (segment (start 67.564 111.252) (end 67.564 120.396) (width 1) (layer B.Cu) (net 40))
 (segment (start 65.846002 101.092) (end 71.21 106.455998) (width 1) (layer B.Cu) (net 40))
 (segment (start 59.113998 101.092) (end 65.846002 101.092) (width 1) (layer B.Cu) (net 40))
 (segment (start 71.21 106.455998) (end 71.21 109.22) (width 1) (layer B.Cu) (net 40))
 (segment (start 57.880001 102.325997) (end 59.113998 101.092) (width 1) (layer B.Cu) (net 40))
 (segment (start 58.48 104.65) (end 57.880001 104.050001) (width 1) (layer B.Cu) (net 40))
 (segment (start 57.880001 104.050001) (end 57.880001 102.325997) (width 1) (layer B.Cu) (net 40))
 (segment (start 62.934 120.904) (end 63.380001 121.350001) (width 0.25) (layer F.Cu) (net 27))
 (segment (start 59.595001 151.543001) (end 57.404 149.352) (width 0.25) (layer F.Cu) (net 27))
 (segment (start 58.42 154.94) (end 59.595001 153.764999) (width 0.25) (layer F.Cu) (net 27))
 (segment (start 63.380001 121.350001) (end 63.98 121.95) (width 0.25) (layer F.Cu) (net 27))
 (segment (start 57.404 149.352) (end 57.404 122.428) (width 0.25) (layer F.Cu) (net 27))
 (segment (start 58.928 120.904) (end 62.934 120.904) (width 0.25) (layer F.Cu) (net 27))
 (segment (start 59.595001 153.764999) (end 59.595001 151.543001) (width 0.25) (layer F.Cu) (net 27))
 (segment (start 57.404 122.428) (end 58.928 120.904) (width 0.25) (layer F.Cu) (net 27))
 (segment (start 68.58 129.032) (end 68.58 114.85) (width 0.25) (layer B.Cu) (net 21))
 (segment (start 50.8 154.94) (end 49.276 153.416) (width 0.25) (layer B.Cu) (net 21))
 (segment (start 68.58 114.85) (end 69.88 113.55) (width 0.25) (layer B.Cu) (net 21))
 (segment (start 49.276 148.336) (end 68.58 129.032) (width 0.25) (layer B.Cu) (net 21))
 (segment (start 49.276 153.416) (end 49.276 148.336) (width 0.25) (layer B.Cu) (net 21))
 (segment (start 71.280001 113.649999) (end 71.88 113.05) (width 0.25) (layer B.Cu) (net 22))
 (segment (start 50.8 152.4) (end 70.866 132.334) (width 0.25) (layer B.Cu) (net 22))
 (segment (start 70.866 114.064) (end 71.280001 113.649999) (width 0.25) (layer B.Cu) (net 22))
 (segment (start 70.866 132.334) (end 70.866 114.064) (width 0.25) (layer B.Cu) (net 22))
 (segment (start 58.0875 95.5525) (end 57.785 95.25) (width 0.25) (layer B.Cu) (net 42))
 (segment (start 58.0875 99.06) (end 58.0875 95.5525) (width 0.25) (layer B.Cu) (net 42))
 (segment (start 53.980001 111.950001) (end 54.58 112.55) (width 0.25) (layer B.Cu) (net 42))
 (segment (start 53.594 111.564) (end 53.980001 111.950001) (width 0.25) (layer B.Cu) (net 42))
 (segment (start 58.0875 99.06) (end 58.039 99.1085) (width 0.25) (layer B.Cu) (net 42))
 (segment (start 53.594 104.521) (end 53.594 111.564) (width 0.25) (layer B.Cu) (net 42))
 (segment (start 58.039 100.076) (end 53.594 104.521) (width 0.25) (layer B.Cu) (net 42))
 (segment (start 58.039 99.1085) (end 58.039 100.076) (width 0.25) (layer B.Cu) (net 42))
 (segment (start 48.26 115.87) (end 50.58 113.55) (width 0.25) (layer B.Cu) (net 24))
 (segment (start 52.164999 153.575001) (end 52.164999 155.860003) (width 0.25) (layer B.Cu) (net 24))
 (segment (start 53.34 152.4) (end 52.164999 153.575001) (width 0.25) (layer B.Cu) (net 24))
 (segment (start 52.164999 155.860003) (end 51.053002 156.972) (width 0.25) (layer B.Cu) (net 24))
 (segment (start 51.053002 156.972) (end 49.276 156.972) (width 0.25) (layer B.Cu) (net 24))
 (segment (start 49.276 156.972) (end 48.26 155.956) (width 0.25) (layer B.Cu) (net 24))
 (segment (start 48.26 155.956) (end 48.26 115.87) (width 0.25) (layer B.Cu) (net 24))
 (segment (start 52.164999 153.764999) (end 52.490001 154.090001) (width 0.25) (layer F.Cu) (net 23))
 (segment (start 55.505001 119.359997) (end 52.164999 122.699999) (width 0.25) (layer F.Cu) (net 23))
 (segment (start 52.164999 122.699999) (end 52.164999 153.764999) (width 0.25) (layer F.Cu) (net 23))
 (segment (start 55.505001 114.975001) (end 55.505001 119.359997) (width 0.25) (layer F.Cu) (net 23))
 (segment (start 52.490001 154.090001) (end 53.34 154.94) (width 0.25) (layer F.Cu) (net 23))
 (segment (start 54.58 114.05) (end 55.505001 114.975001) (width 0.25) (layer F.Cu) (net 23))
 (segment (start 52.4025 95.7325) (end 52.885 95.25) (width 0.25) (layer B.Cu) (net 41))
 (segment (start 52.4025 99.06) (end 52.4025 95.7325) (width 0.25) (layer B.Cu) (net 41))
 (segment (start 51.980001 112.450001) (end 52.58 113.05) (width 0.25) (layer B.Cu) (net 41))
 (segment (start 51.55999 99.90251) (end 51.55999 112.02999) (width 0.25) (layer B.Cu) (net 41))
 (segment (start 51.55999 112.02999) (end 51.980001 112.450001) (width 0.25) (layer B.Cu) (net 41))
 (segment (start 52.4025 99.06) (end 51.55999 99.90251) (width 0.25) (layer B.Cu) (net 41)))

